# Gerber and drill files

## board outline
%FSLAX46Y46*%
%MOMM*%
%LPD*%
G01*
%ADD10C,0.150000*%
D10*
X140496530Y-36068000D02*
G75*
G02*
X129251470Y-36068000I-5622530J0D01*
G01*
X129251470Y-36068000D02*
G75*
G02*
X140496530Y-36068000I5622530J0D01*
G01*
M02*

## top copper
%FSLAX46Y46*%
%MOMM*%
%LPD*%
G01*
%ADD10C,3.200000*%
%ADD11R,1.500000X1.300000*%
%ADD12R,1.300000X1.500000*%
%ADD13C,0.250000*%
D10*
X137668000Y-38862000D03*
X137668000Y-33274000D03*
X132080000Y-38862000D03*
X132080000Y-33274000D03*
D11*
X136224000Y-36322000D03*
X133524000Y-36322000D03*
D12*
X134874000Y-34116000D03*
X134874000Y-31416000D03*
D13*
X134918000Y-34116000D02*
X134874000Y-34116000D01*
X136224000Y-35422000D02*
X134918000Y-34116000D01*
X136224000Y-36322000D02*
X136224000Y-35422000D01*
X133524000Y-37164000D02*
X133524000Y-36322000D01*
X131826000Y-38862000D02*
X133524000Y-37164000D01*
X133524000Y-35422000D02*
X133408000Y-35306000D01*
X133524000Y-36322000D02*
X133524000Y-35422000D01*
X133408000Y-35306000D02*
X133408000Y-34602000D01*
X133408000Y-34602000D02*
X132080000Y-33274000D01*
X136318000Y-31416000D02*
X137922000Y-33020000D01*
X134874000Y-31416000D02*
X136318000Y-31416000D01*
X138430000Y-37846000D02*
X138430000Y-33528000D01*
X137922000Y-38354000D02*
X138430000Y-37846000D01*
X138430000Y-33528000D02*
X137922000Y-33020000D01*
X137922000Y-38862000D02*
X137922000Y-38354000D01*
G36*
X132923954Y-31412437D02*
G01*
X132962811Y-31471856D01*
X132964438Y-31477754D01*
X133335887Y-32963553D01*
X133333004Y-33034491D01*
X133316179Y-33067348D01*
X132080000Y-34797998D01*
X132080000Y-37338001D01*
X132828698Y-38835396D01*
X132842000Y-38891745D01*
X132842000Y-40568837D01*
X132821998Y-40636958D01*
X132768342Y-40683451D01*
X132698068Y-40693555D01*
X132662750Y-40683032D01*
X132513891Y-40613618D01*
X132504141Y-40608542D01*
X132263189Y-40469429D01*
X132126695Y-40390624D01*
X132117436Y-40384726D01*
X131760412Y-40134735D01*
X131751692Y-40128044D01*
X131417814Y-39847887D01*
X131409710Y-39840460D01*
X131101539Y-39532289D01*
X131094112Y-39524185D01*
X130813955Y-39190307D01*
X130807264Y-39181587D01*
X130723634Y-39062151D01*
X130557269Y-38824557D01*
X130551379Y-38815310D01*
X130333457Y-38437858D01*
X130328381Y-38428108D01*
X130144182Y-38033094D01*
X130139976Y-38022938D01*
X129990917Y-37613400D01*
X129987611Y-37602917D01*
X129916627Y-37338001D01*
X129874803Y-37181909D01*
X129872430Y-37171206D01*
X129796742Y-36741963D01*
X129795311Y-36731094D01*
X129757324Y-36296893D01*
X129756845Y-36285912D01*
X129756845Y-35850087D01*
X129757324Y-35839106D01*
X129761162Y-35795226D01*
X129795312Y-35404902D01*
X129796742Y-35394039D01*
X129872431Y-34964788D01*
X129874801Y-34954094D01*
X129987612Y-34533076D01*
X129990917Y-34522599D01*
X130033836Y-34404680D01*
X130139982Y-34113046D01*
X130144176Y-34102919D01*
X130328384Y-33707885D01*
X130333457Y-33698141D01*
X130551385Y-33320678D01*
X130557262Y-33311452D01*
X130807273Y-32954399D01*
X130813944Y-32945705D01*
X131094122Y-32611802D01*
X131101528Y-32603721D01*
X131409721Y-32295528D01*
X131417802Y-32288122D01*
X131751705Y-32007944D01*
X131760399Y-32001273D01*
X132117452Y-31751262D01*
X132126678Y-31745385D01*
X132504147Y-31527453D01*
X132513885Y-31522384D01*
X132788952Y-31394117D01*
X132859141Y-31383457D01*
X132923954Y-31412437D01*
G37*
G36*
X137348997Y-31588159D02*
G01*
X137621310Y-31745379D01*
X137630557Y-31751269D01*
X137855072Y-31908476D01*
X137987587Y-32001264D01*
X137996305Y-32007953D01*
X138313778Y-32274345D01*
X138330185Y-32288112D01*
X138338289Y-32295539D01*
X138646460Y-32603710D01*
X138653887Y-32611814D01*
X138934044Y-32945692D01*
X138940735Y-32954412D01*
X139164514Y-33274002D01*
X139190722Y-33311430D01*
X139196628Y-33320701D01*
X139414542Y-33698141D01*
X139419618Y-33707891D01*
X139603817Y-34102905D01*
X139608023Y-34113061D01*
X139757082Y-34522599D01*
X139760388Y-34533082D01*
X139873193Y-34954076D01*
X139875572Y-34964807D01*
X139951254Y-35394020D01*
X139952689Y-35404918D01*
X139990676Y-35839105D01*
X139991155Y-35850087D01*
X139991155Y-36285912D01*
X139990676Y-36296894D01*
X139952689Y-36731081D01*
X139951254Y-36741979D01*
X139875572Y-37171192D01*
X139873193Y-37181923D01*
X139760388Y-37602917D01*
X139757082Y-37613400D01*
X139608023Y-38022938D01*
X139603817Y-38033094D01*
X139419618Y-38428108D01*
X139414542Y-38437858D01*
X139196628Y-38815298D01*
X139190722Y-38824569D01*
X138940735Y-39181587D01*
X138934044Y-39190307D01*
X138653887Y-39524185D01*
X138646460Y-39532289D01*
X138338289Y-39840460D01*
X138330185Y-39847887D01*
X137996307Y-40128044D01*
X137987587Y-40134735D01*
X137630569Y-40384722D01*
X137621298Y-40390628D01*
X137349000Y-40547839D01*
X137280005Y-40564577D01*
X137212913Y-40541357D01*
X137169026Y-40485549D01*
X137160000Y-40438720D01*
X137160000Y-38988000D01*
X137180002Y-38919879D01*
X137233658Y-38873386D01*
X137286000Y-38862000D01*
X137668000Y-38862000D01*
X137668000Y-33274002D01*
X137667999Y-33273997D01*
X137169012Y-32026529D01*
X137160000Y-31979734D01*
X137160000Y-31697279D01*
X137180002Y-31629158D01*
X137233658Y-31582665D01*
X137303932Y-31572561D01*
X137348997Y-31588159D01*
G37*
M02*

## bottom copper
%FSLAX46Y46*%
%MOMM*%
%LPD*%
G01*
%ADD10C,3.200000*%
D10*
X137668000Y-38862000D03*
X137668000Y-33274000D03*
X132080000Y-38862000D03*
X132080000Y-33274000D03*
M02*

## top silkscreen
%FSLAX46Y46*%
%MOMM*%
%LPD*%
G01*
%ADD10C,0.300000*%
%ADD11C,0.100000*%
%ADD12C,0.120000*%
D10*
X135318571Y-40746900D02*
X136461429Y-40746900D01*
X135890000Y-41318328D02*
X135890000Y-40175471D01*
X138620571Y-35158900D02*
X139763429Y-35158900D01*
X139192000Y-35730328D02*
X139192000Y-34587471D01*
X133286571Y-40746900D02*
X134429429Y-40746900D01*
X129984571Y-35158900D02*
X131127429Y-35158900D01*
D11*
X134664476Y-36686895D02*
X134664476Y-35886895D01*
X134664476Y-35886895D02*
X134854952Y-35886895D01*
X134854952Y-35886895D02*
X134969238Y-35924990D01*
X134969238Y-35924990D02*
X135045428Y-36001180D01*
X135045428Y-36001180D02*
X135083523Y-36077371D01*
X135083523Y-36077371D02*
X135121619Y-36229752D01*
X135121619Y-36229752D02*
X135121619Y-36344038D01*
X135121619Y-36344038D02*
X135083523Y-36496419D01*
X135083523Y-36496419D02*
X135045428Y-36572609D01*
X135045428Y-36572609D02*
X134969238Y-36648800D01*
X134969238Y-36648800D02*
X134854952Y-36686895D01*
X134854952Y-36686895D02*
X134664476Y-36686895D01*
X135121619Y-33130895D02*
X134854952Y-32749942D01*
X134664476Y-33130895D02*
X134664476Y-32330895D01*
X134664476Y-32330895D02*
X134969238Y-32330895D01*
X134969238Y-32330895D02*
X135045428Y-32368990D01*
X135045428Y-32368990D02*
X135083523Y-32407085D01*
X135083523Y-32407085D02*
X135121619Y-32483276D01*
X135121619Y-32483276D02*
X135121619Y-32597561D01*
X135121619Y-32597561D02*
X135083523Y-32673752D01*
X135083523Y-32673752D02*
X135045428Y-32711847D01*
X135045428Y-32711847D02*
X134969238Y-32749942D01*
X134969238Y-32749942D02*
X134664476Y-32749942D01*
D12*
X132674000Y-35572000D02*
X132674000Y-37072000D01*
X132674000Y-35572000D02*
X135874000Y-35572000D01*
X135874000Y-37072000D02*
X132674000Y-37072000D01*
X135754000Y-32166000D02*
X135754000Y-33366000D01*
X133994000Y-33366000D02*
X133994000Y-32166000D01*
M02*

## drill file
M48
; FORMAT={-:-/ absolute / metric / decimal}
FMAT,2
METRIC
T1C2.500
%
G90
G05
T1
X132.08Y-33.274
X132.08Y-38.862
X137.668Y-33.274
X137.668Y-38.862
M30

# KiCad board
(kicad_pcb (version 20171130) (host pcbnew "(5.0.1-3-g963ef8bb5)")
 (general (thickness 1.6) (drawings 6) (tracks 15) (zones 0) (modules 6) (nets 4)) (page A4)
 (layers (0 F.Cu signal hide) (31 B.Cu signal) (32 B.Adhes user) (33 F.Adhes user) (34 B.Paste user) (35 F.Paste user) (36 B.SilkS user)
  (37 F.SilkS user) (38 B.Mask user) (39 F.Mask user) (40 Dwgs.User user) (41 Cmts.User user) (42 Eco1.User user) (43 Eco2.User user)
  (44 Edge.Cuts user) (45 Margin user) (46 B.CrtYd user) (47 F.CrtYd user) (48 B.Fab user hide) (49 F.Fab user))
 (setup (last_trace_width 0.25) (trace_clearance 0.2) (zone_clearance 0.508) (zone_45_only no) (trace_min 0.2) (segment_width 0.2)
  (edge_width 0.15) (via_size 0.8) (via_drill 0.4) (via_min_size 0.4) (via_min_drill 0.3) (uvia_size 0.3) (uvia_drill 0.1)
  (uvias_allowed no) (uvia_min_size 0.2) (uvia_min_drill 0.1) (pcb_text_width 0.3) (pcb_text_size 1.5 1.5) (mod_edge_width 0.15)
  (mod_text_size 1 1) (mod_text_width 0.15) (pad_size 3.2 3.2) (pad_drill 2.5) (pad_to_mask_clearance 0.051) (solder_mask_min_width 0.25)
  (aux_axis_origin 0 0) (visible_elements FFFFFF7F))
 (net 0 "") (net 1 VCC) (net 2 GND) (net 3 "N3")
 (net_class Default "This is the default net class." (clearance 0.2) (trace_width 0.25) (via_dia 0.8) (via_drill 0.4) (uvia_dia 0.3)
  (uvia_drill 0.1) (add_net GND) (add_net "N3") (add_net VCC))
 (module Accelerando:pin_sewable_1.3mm (layer F.Cu) (at 137.668 38.862)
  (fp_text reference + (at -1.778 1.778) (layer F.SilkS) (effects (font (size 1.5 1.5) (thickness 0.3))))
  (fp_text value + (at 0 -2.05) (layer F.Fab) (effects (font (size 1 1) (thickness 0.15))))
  (pad 1 thru_hole circle (at 0 0) (size 3.2 3.2) (drill 2.5) (layers *.Cu *.Mask) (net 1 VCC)))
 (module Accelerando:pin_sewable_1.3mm (layer F.Cu) (at 137.668 33.274)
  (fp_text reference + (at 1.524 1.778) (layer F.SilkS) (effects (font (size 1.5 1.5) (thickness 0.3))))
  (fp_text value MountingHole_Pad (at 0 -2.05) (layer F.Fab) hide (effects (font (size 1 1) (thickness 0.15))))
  (pad 1 thru_hole circle (at 0 0) (size 3.2 3.2) (drill 2.5) (layers *.Cu *.Mask) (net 1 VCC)))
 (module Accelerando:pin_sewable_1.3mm (layer F.Cu) (at 132.08 38.862)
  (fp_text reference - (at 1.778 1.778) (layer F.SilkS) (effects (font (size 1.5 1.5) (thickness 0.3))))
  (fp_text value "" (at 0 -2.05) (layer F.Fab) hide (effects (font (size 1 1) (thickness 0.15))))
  (pad 1 thru_hole circle (at 0 0) (size 3.2 3.2) (drill 2.5) (layers *.Cu *.Mask) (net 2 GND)))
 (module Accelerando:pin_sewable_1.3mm (layer F.Cu) (at 132.08 33.274)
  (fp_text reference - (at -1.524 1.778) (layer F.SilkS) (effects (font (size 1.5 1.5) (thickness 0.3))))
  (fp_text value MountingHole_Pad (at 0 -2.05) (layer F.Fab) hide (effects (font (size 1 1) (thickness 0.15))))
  (pad 1 thru_hole circle (at 0 0) (size 3.2 3.2) (drill 2.5) (layers *.Cu *.Mask) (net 2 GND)))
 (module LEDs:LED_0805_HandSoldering (layer F.Cu) (at 134.874 36.322)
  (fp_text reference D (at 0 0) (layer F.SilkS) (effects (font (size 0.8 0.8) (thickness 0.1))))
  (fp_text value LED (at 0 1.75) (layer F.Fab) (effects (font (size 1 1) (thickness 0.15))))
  (fp_line (start -2.2 -0.75) (end -2.2 0.75) (layer F.SilkS) (width 0.12))
  (fp_line (start -2.2 -0.75) (end 1 -0.75) (layer F.SilkS) (width 0.12))
  (fp_line (start 1 0.75) (end -2.2 0.75) (layer F.SilkS) (width 0.12))
  (pad 2 smd rect (at 1.35 0) (size 1.5 1.3) (layers F.Cu F.Paste F.Mask) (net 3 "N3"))
  (pad 1 smd rect (at -1.35 0) (size 1.5 1.3) (layers F.Cu F.Paste F.Mask) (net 2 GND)))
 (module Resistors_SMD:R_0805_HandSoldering (layer F.Cu) (at 134.874 32.766 270)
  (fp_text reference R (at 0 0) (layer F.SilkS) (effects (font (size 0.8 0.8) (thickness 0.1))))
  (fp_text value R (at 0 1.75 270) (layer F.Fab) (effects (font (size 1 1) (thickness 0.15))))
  (fp_line (start -0.6 -0.88) (end 0.6 -0.88) (layer F.SilkS) (width 0.12))
  (fp_line (start 0.6 0.88) (end -0.6 0.88) (layer F.SilkS) (width 0.12))
  (pad 2 smd rect (at 1.35 0 270) (size 1.5 1.3) (layers F.Cu F.Paste F.Mask) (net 3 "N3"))
  (pad 1 smd rect (at -1.35 0 270) (size 1.5 1.3) (layers F.Cu F.Paste F.Mask) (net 1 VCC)))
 (gr_circle (center 134.874 36.068) (end 140.208 37.846) (layer Edge.Cuts) (width 0.15))
 (segment (start 134.918 34.116) (end 134.874 34.116) (width 0.25) (layer F.Cu) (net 3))
 (segment (start 136.224 35.422) (end 134.918 34.116) (width 0.25) (layer F.Cu) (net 3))
 (segment (start 136.224 36.322) (end 136.224 35.422) (width 0.25) (layer F.Cu) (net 3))
 (segment (start 133.524 37.164) (end 133.524 36.322) (width 0.25) (layer F.Cu) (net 2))
 (segment (start 131.826 38.862) (end 133.524 37.164) (width 0.25) (layer F.Cu) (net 2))
 (segment (start 133.524 35.422) (end 133.408 35.306) (width 0.25) (layer F.Cu) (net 2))
 (segment (start 133.524 36.322) (end 133.524 35.422) (width 0.25) (layer F.Cu) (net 2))
 (segment (start 133.408 35.306) (end 133.408 34.602) (width 0.25) (layer F.Cu) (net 2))
 (segment (start 133.408 34.602) (end 132.08 33.274) (width 0.25) (layer F.Cu) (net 2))
 (segment (start 136.318 31.416) (end 137.922 33.02) (width 0.25) (layer F.Cu) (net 1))
 (segment (start 134.874 31.416) (end 136.318 31.416) (width 0.25) (layer F.Cu) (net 1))
 (segment (start 138.43 37.846) (end 138.43 33.528) (width 0.25) (layer F.Cu) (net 1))
 (segment (start 137.922 38.354) (end 138.43 37.846) (width 0.25) (layer F.Cu) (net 1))
 (segment (start 138.43 33.528) (end 137.922 33.02) (width 0.25) (layer F.Cu) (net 1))
 (segment (start 137.922 38.862) (end 137.922 38.354) (width 0.25) (layer F.Cu) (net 1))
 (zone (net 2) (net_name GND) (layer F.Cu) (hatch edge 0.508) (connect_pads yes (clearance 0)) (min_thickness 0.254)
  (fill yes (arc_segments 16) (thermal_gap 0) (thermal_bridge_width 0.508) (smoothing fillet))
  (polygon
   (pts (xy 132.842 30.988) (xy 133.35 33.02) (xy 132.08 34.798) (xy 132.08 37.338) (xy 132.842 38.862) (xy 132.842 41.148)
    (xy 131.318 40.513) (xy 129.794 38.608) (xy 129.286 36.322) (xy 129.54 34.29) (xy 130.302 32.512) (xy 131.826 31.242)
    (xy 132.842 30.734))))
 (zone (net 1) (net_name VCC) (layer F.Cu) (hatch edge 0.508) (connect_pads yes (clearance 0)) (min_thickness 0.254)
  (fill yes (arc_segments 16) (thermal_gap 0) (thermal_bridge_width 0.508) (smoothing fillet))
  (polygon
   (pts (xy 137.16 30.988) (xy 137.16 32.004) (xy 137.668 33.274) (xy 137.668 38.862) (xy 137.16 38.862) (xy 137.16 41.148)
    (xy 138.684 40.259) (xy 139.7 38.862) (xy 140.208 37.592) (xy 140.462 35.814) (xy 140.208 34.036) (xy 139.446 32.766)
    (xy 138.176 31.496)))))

